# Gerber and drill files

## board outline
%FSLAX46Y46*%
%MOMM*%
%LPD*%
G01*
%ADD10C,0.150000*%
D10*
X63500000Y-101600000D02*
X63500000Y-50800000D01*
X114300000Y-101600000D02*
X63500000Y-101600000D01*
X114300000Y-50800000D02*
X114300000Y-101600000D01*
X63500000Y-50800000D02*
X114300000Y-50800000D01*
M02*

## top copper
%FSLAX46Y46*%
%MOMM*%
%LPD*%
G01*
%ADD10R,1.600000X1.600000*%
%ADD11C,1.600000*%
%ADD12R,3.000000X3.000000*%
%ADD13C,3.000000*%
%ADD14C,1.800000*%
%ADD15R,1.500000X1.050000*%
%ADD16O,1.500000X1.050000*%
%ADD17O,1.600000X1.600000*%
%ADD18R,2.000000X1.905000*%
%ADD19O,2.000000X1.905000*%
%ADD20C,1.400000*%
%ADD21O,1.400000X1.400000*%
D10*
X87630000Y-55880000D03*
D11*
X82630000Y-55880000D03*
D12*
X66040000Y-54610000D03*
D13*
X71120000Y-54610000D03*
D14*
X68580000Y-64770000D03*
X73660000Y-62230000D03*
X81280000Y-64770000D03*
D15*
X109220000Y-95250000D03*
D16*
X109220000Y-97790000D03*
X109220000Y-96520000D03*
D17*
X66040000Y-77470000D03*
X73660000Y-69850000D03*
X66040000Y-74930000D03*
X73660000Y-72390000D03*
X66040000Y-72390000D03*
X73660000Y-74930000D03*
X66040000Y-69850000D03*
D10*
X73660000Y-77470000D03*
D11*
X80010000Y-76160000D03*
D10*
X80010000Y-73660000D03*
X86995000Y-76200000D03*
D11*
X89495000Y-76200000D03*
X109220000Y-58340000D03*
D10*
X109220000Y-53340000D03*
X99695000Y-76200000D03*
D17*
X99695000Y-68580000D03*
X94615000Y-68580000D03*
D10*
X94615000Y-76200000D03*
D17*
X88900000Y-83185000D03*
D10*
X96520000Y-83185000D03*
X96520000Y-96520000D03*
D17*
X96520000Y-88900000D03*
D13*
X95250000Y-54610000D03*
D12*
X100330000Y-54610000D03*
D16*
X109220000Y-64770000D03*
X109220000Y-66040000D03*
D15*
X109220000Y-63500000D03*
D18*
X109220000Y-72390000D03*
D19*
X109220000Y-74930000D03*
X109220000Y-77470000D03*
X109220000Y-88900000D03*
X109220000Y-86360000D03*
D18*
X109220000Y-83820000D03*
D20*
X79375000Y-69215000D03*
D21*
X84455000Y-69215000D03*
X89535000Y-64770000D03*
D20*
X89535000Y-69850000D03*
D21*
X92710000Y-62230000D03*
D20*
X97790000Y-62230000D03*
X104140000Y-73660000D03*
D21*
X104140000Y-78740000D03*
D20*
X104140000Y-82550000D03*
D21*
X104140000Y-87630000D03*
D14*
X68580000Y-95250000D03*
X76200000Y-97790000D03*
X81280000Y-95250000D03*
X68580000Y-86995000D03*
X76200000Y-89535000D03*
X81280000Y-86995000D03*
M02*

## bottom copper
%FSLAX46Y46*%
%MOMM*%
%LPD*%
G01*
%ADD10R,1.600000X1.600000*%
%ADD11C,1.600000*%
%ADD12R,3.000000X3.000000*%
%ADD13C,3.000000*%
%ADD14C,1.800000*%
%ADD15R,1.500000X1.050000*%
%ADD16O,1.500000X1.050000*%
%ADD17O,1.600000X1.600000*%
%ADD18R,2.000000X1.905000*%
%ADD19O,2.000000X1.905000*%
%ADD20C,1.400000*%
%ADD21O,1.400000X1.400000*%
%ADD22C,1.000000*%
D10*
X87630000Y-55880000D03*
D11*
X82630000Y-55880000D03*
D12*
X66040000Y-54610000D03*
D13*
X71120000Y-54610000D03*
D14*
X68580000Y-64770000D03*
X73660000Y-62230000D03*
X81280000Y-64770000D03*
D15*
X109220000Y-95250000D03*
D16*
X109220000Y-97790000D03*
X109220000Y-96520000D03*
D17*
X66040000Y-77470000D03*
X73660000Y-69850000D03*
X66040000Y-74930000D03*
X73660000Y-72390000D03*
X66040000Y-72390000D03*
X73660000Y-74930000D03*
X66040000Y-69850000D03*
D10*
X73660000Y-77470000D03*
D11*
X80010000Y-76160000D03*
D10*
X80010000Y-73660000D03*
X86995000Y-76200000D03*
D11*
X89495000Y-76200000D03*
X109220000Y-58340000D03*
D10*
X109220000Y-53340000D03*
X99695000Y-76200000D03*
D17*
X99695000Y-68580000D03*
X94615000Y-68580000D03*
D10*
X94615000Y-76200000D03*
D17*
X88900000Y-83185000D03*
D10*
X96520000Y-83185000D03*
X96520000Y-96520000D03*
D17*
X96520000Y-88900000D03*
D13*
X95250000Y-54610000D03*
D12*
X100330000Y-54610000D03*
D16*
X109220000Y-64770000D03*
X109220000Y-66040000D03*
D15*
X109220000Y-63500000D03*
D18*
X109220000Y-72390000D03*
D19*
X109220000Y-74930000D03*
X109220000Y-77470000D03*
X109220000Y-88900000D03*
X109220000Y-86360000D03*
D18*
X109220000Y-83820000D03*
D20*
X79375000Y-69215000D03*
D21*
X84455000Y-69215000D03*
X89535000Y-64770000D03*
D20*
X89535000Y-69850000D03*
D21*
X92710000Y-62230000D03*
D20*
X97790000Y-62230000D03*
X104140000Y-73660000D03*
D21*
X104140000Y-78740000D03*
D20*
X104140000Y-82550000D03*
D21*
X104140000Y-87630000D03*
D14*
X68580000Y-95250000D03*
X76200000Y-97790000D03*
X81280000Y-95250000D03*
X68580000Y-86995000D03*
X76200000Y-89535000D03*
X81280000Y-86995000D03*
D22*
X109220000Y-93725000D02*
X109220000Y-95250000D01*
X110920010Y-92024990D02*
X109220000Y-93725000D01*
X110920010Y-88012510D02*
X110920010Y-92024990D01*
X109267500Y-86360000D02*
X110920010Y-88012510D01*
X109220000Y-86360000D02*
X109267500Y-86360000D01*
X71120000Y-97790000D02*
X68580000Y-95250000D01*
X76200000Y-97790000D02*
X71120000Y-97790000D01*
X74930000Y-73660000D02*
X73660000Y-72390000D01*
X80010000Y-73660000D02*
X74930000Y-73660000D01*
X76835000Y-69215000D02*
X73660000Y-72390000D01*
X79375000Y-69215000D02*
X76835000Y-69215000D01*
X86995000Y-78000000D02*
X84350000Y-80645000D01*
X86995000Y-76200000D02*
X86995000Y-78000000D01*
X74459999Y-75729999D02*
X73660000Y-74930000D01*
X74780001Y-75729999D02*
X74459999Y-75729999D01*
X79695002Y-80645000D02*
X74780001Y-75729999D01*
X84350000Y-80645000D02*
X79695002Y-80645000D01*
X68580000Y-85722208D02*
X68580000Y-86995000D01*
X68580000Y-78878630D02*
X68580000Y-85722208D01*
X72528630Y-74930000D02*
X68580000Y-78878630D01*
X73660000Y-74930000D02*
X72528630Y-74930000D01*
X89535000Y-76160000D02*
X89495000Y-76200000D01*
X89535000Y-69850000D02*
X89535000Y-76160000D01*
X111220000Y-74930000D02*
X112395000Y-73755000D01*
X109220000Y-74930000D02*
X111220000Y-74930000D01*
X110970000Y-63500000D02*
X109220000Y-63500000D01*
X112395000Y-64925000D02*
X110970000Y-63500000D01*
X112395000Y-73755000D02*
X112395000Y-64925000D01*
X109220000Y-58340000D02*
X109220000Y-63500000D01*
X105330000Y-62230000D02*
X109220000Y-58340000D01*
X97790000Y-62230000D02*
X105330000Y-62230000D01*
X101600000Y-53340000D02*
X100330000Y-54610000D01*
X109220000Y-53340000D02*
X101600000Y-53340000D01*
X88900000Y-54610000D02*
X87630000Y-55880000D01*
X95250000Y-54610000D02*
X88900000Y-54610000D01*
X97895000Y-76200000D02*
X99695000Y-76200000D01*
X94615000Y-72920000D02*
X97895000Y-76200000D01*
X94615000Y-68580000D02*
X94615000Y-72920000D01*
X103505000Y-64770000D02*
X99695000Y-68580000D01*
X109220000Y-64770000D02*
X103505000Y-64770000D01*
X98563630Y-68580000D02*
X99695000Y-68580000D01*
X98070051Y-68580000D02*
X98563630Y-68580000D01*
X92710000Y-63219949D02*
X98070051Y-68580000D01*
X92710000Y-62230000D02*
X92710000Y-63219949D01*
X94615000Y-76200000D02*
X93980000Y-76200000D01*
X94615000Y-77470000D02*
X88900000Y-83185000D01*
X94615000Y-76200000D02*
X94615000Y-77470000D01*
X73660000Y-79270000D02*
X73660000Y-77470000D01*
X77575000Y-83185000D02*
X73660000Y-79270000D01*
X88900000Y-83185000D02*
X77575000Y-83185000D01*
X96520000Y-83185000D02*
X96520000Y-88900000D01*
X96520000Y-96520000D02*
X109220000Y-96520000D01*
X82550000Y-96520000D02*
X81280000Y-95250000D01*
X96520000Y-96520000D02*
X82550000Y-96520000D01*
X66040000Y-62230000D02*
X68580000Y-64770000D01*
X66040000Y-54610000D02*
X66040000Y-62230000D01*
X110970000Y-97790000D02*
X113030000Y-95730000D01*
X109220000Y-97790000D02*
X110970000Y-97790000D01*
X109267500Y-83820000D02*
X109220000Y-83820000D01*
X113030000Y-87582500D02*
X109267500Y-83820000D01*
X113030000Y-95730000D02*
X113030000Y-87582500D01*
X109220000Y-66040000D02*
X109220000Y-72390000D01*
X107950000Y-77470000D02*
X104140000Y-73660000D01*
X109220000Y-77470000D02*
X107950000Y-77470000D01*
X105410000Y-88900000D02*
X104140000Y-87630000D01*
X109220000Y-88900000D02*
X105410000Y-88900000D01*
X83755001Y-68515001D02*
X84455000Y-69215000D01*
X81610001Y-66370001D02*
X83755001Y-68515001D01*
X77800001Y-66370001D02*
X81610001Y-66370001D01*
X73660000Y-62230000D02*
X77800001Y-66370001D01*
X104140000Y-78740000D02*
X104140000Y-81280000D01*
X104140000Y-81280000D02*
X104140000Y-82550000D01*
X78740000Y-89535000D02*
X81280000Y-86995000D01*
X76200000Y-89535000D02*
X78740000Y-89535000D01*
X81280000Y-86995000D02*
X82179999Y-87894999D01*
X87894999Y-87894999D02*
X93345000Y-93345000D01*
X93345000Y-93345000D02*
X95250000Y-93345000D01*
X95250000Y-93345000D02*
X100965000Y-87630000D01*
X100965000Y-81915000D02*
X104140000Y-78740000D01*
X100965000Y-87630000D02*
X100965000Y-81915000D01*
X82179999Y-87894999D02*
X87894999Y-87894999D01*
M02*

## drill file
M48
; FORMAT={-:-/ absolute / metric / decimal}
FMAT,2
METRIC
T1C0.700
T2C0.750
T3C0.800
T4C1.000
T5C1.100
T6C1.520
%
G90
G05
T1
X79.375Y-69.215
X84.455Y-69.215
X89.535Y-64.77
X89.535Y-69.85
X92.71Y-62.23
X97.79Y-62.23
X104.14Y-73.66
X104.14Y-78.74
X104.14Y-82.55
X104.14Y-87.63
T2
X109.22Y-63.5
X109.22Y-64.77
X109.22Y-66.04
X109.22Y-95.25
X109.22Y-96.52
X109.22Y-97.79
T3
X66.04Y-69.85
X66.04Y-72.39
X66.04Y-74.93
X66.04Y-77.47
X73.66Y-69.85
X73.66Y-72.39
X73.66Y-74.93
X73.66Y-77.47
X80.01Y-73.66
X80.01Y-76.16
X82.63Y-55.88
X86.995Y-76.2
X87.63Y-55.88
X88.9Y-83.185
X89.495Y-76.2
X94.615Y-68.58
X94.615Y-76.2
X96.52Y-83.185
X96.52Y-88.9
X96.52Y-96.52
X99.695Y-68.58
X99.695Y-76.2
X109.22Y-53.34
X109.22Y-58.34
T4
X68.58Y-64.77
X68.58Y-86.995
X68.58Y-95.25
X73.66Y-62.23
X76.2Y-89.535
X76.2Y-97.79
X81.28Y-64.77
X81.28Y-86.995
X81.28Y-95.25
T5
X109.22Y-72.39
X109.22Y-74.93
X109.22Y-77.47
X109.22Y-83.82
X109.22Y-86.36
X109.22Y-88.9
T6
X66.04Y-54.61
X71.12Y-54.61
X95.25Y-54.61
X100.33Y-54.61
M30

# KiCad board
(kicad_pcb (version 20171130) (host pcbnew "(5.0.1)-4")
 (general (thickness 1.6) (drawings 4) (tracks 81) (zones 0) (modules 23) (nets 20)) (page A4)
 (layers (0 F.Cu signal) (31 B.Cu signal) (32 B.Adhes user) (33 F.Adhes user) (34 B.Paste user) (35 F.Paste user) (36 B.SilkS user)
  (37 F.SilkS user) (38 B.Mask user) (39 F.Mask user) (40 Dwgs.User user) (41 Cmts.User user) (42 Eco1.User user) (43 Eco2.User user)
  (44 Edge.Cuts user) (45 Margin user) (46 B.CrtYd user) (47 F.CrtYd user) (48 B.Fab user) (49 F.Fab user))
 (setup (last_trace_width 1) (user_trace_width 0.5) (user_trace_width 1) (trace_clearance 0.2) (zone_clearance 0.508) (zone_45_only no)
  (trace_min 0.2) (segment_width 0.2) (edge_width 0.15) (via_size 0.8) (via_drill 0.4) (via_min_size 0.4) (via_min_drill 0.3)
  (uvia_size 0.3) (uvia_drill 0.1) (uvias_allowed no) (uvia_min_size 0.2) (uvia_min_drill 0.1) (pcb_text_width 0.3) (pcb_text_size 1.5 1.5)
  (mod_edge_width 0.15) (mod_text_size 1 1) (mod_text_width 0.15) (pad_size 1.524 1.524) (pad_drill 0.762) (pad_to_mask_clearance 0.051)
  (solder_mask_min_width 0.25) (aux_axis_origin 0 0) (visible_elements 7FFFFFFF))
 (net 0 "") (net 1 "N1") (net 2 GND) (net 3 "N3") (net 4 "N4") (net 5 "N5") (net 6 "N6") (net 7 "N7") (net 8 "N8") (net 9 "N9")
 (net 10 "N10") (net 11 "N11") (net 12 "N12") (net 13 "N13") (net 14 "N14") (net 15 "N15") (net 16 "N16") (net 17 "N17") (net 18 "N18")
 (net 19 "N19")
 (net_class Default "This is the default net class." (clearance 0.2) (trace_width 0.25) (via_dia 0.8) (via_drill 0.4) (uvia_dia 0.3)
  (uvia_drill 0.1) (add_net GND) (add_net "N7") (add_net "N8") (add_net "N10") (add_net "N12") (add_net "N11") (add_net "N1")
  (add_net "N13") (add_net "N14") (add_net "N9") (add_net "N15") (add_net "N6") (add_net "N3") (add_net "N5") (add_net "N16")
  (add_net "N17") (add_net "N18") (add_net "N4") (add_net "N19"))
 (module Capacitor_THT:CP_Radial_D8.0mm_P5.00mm (layer F.Cu) (at 87.63 55.88 180)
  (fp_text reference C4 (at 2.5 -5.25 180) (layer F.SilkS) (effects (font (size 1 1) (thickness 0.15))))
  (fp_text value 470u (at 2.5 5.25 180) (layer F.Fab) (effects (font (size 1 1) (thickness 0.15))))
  (pad 1 thru_hole rect (at 0 0 180) (size 1.6 1.6) (drill 0.8) (layers *.Cu *.Mask) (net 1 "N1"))
  (pad 2 thru_hole circle (at 5 0 180) (size 1.6 1.6) (drill 0.8) (layers *.Cu *.Mask) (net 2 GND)))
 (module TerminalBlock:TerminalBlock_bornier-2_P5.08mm (layer F.Cu) (at 66.04 54.61)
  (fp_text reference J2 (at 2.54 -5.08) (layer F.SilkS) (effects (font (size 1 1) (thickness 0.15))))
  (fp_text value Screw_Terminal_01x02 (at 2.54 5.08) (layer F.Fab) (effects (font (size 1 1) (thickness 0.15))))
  (pad 1 thru_hole rect (at 0 0) (size 3 3) (drill 1.52) (layers *.Cu *.Mask) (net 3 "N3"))
  (pad 2 thru_hole circle (at 5.08 0) (size 3 3) (drill 1.52) (layers *.Cu *.Mask) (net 2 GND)))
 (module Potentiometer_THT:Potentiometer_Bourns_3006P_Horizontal (layer F.Cu) (at 81.28 64.77)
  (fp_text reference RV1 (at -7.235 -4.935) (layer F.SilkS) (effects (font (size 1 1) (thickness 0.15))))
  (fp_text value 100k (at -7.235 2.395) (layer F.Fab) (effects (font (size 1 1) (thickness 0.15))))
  (pad 3 thru_hole circle (at -12.7 0) (size 1.8 1.8) (drill 1) (layers *.Cu *.Mask) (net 3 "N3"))
  (pad 2 thru_hole circle (at -7.62 -2.54) (size 1.8 1.8) (drill 1) (layers *.Cu *.Mask) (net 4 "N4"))
  (pad 1 thru_hole circle (at 0 0) (size 1.8 1.8) (drill 1) (layers *.Cu *.Mask) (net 2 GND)))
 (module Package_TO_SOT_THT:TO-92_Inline (layer F.Cu) (at 109.22 95.25 270)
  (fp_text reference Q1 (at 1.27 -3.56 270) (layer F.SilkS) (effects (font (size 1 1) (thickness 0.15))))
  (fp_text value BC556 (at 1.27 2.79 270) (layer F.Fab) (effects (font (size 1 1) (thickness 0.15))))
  (pad 1 thru_hole rect (at 0 0 270) (size 1.05 1.5) (drill 0.75) (layers *.Cu *.Mask) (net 2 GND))
  (pad 3 thru_hole oval (at 2.54 0 270) (size 1.05 1.5) (drill 0.75) (layers *.Cu *.Mask) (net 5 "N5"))
  (pad 2 thru_hole oval (at 1.27 0 270) (size 1.05 1.5) (drill 0.75) (layers *.Cu *.Mask) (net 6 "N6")))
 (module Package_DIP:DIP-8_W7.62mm (layer F.Cu) (at 73.66 77.47 180)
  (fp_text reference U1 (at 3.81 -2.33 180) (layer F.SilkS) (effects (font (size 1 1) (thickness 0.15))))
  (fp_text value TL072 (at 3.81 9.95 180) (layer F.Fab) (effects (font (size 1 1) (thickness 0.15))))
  (pad 8 thru_hole oval (at 7.62 0 180) (size 1.6 1.6) (drill 0.8) (layers *.Cu *.Mask))
  (pad 4 thru_hole oval (at 0 7.62 180) (size 1.6 1.6) (drill 0.8) (layers *.Cu *.Mask))
  (pad 7 thru_hole oval (at 7.62 2.54 180) (size 1.6 1.6) (drill 0.8) (layers *.Cu *.Mask))
  (pad 3 thru_hole oval (at 0 5.08 180) (size 1.6 1.6) (drill 0.8) (layers *.Cu *.Mask) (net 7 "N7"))
  (pad 6 thru_hole oval (at 7.62 5.08 180) (size 1.6 1.6) (drill 0.8) (layers *.Cu *.Mask))
  (pad 2 thru_hole oval (at 0 2.54 180) (size 1.6 1.6) (drill 0.8) (layers *.Cu *.Mask) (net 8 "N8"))
  (pad 5 thru_hole oval (at 7.62 7.62 180) (size 1.6 1.6) (drill 0.8) (layers *.Cu *.Mask))
  (pad 1 thru_hole rect (at 0 0 180) (size 1.6 1.6) (drill 0.8) (layers *.Cu *.Mask) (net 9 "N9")))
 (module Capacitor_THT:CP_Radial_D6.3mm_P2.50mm (layer F.Cu) (at 80.01 73.66 270)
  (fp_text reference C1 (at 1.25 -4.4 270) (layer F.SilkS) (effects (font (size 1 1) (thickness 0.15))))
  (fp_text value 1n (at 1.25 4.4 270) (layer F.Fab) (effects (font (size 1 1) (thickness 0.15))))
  (pad 2 thru_hole circle (at 2.5 0 270) (size 1.6 1.6) (drill 0.8) (layers *.Cu *.Mask) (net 2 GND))
  (pad 1 thru_hole rect (at 0 0 270) (size 1.6 1.6) (drill 0.8) (layers *.Cu *.Mask) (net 7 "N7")))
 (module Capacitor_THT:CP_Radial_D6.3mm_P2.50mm (layer F.Cu) (at 86.995 76.2)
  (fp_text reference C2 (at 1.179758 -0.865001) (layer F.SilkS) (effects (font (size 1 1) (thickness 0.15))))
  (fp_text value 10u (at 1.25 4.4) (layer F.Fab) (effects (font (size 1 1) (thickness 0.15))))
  (pad 1 thru_hole rect (at 0 0) (size 1.6 1.6) (drill 0.8) (layers *.Cu *.Mask) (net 8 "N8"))
  (pad 2 thru_hole circle (at 2.5 0) (size 1.6 1.6) (drill 0.8) (layers *.Cu *.Mask) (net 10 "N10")))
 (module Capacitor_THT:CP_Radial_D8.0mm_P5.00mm (layer F.Cu) (at 109.22 53.34 270)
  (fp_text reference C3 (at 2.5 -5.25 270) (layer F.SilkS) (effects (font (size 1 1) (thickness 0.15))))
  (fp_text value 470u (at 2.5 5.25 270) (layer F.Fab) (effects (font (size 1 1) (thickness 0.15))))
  (pad 2 thru_hole circle (at 5 0 270) (size 1.6 1.6) (drill 0.8) (layers *.Cu *.Mask) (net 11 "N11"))
  (pad 1 thru_hole rect (at 0 0 270) (size 1.6 1.6) (drill 0.8) (layers *.Cu *.Mask) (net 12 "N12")))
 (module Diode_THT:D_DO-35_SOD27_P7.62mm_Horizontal (layer F.Cu) (at 99.695 76.2 90)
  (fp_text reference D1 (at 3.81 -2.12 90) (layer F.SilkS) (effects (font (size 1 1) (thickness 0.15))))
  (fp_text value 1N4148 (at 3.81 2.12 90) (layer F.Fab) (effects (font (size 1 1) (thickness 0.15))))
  (pad 1 thru_hole rect (at 0 0 90) (size 1.6 1.6) (drill 0.8) (layers *.Cu *.Mask) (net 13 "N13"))
  (pad 2 thru_hole oval (at 7.62 0 90) (size 1.6 1.6) (drill 0.8) (layers *.Cu *.Mask) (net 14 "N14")))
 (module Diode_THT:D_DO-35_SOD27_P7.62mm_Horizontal (layer F.Cu) (at 94.615 76.2 90)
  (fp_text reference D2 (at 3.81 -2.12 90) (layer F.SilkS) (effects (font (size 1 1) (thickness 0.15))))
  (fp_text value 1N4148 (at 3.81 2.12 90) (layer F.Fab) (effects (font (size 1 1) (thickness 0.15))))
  (pad 2 thru_hole oval (at 7.62 0 90) (size 1.6 1.6) (drill 0.8) (layers *.Cu *.Mask) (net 13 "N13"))
  (pad 1 thru_hole rect (at 0 0 90) (size 1.6 1.6) (drill 0.8) (layers *.Cu *.Mask) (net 9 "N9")))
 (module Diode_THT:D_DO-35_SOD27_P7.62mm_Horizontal (layer F.Cu) (at 96.52 83.185 180)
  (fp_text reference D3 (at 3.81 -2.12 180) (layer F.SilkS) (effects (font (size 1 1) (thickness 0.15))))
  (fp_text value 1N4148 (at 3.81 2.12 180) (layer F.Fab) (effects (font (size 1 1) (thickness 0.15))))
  (pad 2 thru_hole oval (at 7.62 0 180) (size 1.6 1.6) (drill 0.8) (layers *.Cu *.Mask) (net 9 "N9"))
  (pad 1 thru_hole rect (at 0 0 180) (size 1.6 1.6) (drill 0.8) (layers *.Cu *.Mask) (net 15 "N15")))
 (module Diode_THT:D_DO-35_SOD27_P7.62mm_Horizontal (layer F.Cu) (at 96.52 96.52 90)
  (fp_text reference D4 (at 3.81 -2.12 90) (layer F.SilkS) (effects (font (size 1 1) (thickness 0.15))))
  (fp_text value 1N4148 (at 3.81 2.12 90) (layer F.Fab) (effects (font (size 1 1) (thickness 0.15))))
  (pad 1 thru_hole rect (at 0 0 90) (size 1.6 1.6) (drill 0.8) (layers *.Cu *.Mask) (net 6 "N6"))
  (pad 2 thru_hole oval (at 7.62 0 90) (size 1.6 1.6) (drill 0.8) (layers *.Cu *.Mask) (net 15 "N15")))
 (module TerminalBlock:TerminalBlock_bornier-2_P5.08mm (layer F.Cu) (at 100.33 54.61 180)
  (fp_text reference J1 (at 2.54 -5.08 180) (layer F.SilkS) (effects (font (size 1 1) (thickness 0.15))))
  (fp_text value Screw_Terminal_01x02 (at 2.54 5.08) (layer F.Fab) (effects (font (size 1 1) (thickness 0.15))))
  (pad 2 thru_hole circle (at 5.08 0 180) (size 3 3) (drill 1.52) (layers *.Cu *.Mask) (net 1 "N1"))
  (pad 1 thru_hole rect (at 0 0 180) (size 3 3) (drill 1.52) (layers *.Cu *.Mask) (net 12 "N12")))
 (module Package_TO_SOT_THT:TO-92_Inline (layer F.Cu) (at 109.22 63.5 270)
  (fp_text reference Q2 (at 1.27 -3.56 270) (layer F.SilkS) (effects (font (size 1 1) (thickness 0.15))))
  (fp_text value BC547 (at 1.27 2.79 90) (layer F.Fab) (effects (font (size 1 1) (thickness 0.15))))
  (pad 2 thru_hole oval (at 1.27 0 270) (size 1.05 1.5) (drill 0.75) (layers *.Cu *.Mask) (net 14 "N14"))
  (pad 3 thru_hole oval (at 2.54 0 270) (size 1.05 1.5) (drill 0.75) (layers *.Cu *.Mask) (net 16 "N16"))
  (pad 1 thru_hole rect (at 0 0 270) (size 1.05 1.5) (drill 0.75) (layers *.Cu *.Mask) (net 11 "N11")))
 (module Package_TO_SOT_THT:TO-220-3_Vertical (layer F.Cu) (at 109.22 72.39 270)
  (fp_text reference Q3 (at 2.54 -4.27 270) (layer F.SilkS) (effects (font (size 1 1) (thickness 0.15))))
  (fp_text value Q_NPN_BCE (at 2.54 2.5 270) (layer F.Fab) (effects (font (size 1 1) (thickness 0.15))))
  (pad 1 thru_hole rect (at 0 0 270) (size 1.905 2) (drill 1.1) (layers *.Cu *.Mask) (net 16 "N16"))
  (pad 2 thru_hole oval (at 2.54 0 270) (size 1.905 2) (drill 1.1) (layers *.Cu *.Mask) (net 11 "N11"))
  (pad 3 thru_hole oval (at 5.08 0 270) (size 1.905 2) (drill 1.1) (layers *.Cu *.Mask) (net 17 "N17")))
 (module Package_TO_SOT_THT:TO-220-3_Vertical (layer F.Cu) (at 109.22 83.82 270)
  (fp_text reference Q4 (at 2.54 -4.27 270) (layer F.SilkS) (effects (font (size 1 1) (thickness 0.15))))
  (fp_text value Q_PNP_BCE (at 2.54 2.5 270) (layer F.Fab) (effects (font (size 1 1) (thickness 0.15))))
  (pad 3 thru_hole oval (at 5.08 0 270) (size 1.905 2) (drill 1.1) (layers *.Cu *.Mask) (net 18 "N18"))
  (pad 2 thru_hole oval (at 2.54 0 270) (size 1.905 2) (drill 1.1) (layers *.Cu *.Mask) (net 2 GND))
  (pad 1 thru_hole rect (at 0 0 270) (size 1.905 2) (drill 1.1) (layers *.Cu *.Mask) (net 5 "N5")))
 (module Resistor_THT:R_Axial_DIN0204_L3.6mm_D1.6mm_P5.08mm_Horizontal (layer F.Cu) (at 79.375 69.215)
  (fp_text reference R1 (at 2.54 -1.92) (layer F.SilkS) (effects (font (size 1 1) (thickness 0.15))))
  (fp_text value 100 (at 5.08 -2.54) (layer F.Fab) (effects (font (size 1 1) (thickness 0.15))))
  (pad 1 thru_hole circle (at 0 0) (size 1.4 1.4) (drill 0.7) (layers *.Cu *.Mask) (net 7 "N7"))
  (pad 2 thru_hole oval (at 5.08 0) (size 1.4 1.4) (drill 0.7) (layers *.Cu *.Mask) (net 4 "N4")))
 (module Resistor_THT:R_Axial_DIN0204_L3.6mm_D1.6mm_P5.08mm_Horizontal (layer F.Cu) (at 89.535 69.85 90)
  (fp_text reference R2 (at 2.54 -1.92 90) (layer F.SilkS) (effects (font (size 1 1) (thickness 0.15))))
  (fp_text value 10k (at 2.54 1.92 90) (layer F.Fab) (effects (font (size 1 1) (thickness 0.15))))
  (pad 2 thru_hole oval (at 5.08 0 90) (size 1.4 1.4) (drill 0.7) (layers *.Cu *.Mask) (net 2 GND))
  (pad 1 thru_hole circle (at 0 0 90) (size 1.4 1.4) (drill 0.7) (layers *.Cu *.Mask) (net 10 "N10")))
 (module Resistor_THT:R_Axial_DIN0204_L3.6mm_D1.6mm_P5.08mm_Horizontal (layer F.Cu) (at 97.79 62.23 180)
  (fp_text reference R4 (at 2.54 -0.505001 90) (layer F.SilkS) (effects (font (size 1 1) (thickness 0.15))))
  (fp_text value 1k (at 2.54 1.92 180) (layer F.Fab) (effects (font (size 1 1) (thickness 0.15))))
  (pad 2 thru_hole oval (at 5.08 0 180) (size 1.4 1.4) (drill 0.7) (layers *.Cu *.Mask) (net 14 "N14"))
  (pad 1 thru_hole circle (at 0 0 180) (size 1.4 1.4) (drill 0.7) (layers *.Cu *.Mask) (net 11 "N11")))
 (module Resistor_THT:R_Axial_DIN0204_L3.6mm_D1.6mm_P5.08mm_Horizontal (layer F.Cu) (at 104.14 73.66 270)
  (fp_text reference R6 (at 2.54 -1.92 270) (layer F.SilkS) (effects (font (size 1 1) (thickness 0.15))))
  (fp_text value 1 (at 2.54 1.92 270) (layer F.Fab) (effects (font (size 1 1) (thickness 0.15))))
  (pad 1 thru_hole circle (at 0 0 270) (size 1.4 1.4) (drill 0.7) (layers *.Cu *.Mask) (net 17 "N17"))
  (pad 2 thru_hole oval (at 5.08 0 270) (size 1.4 1.4) (drill 0.7) (layers *.Cu *.Mask) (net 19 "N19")))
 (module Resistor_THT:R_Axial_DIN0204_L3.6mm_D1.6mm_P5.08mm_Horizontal (layer F.Cu) (at 104.14 82.55 270)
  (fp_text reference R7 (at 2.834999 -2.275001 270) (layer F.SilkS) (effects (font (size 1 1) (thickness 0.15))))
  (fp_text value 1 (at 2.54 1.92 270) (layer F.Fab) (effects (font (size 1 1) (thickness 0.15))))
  (pad 1 thru_hole circle (at 0 0 270) (size 1.4 1.4) (drill 0.7) (layers *.Cu *.Mask) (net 19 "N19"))
  (pad 2 thru_hole oval (at 5.08 0 270) (size 1.4 1.4) (drill 0.7) (layers *.Cu *.Mask) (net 18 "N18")))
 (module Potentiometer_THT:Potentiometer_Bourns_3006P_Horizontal (layer F.Cu) (at 68.58 95.25 180)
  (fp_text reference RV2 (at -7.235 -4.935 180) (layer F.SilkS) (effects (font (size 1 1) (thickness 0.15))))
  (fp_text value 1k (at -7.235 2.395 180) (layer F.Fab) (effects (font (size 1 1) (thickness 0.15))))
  (pad 1 thru_hole circle (at 0 0 180) (size 1.8 1.8) (drill 1) (layers *.Cu *.Mask) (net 2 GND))
  (pad 2 thru_hole circle (at -7.62 -2.54 180) (size 1.8 1.8) (drill 1) (layers *.Cu *.Mask) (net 2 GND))
  (pad 3 thru_hole circle (at -12.7 0 180) (size 1.8 1.8) (drill 1) (layers *.Cu *.Mask) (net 6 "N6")))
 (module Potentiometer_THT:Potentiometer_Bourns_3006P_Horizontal (layer F.Cu) (at 68.58 86.995 180)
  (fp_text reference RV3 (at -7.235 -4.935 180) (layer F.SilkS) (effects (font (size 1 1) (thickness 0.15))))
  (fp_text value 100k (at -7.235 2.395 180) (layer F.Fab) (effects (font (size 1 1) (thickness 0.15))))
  (pad 1 thru_hole circle (at 0 0 180) (size 1.8 1.8) (drill 1) (layers *.Cu *.Mask) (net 8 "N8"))
  (pad 2 thru_hole circle (at -7.62 -2.54 180) (size 1.8 1.8) (drill 1) (layers *.Cu *.Mask) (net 19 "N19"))
  (pad 3 thru_hole circle (at -12.7 0 180) (size 1.8 1.8) (drill 1) (layers *.Cu *.Mask) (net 19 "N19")))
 (gr_line (start 63.5 101.6) (end 63.5 50.8) (layer Edge.Cuts) (width 0.15))
 (gr_line (start 114.3 101.6) (end 63.5 101.6) (layer Edge.Cuts) (width 0.15))
 (gr_line (start 114.3 50.8) (end 114.3 101.6) (layer Edge.Cuts) (width 0.15))
 (gr_line (start 63.5 50.8) (end 114.3 50.8) (layer Edge.Cuts) (width 0.15))
 (segment (start 109.22 93.725) (end 109.22 95.25) (width 1) (layer B.Cu) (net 2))
 (segment (start 110.92001 92.02499) (end 109.22 93.725) (width 1) (layer B.Cu) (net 2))
 (segment (start 110.92001 88.01251) (end 110.92001 92.02499) (width 1) (layer B.Cu) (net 2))
 (segment (start 109.2675 86.36) (end 110.92001 88.01251) (width 1) (layer B.Cu) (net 2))
 (segment (start 109.22 86.36) (end 109.2675 86.36) (width 1) (layer B.Cu) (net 2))
 (segment (start 71.12 97.79) (end 68.58 95.25) (width 1) (layer B.Cu) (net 2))
 (segment (start 76.2 97.79) (end 71.12 97.79) (width 1) (layer B.Cu) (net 2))
 (segment (start 74.93 73.66) (end 73.66 72.39) (width 1) (layer B.Cu) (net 7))
 (segment (start 80.01 73.66) (end 74.93 73.66) (width 1) (layer B.Cu) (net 7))
 (segment (start 76.835 69.215) (end 73.66 72.39) (width 1) (layer B.Cu) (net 7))
 (segment (start 79.375 69.215) (end 76.835 69.215) (width 1) (layer B.Cu) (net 7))
 (segment (start 86.995 78) (end 84.35 80.645) (width 1) (layer B.Cu) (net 8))
 (segment (start 86.995 76.2) (end 86.995 78) (width 1) (layer B.Cu) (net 8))
 (segment (start 74.459999 75.729999) (end 73.66 74.93) (width 1) (layer B.Cu) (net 8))
 (segment (start 74.780001 75.729999) (end 74.459999 75.729999) (width 1) (layer B.Cu) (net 8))
 (segment (start 79.695002 80.645) (end 74.780001 75.729999) (width 1) (layer B.Cu) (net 8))
 (segment (start 84.35 80.645) (end 79.695002 80.645) (width 1) (layer B.Cu) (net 8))
 (segment (start 68.58 85.722208) (end 68.58 86.995) (width 1) (layer B.Cu) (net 8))
 (segment (start 68.58 78.87863) (end 68.58 85.722208) (width 1) (layer B.Cu) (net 8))
 (segment (start 72.52863 74.93) (end 68.58 78.87863) (width 1) (layer B.Cu) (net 8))
 (segment (start 73.66 74.93) (end 72.52863 74.93) (width 1) (layer B.Cu) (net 8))
 (segment (start 89.535 76.16) (end 89.495 76.2) (width 1) (layer B.Cu) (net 10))
 (segment (start 89.535 69.85) (end 89.535 76.16) (width 1) (layer B.Cu) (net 10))
 (segment (start 111.22 74.93) (end 112.395 73.755) (width 1) (layer B.Cu) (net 11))
 (segment (start 109.22 74.93) (end 111.22 74.93) (width 1) (layer B.Cu) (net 11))
 (segment (start 110.97 63.5) (end 109.22 63.5) (width 1) (layer B.Cu) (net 11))
 (segment (start 112.395 64.925) (end 110.97 63.5) (width 1) (layer B.Cu) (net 11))
 (segment (start 112.395 73.755) (end 112.395 64.925) (width 1) (layer B.Cu) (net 11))
 (segment (start 109.22 58.34) (end 109.22 63.5) (width 1) (layer B.Cu) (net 11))
 (segment (start 105.33 62.23) (end 109.22 58.34) (width 1) (layer B.Cu) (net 11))
 (segment (start 97.79 62.23) (end 105.33 62.23) (width 1) (layer B.Cu) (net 11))
 (segment (start 101.6 53.34) (end 100.33 54.61) (width 1) (layer B.Cu) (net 12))
 (segment (start 109.22 53.34) (end 101.6 53.34) (width 1) (layer B.Cu) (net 12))
 (segment (start 88.9 54.61) (end 87.63 55.88) (width 1) (layer B.Cu) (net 1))
 (segment (start 95.25 54.61) (end 88.9 54.61) (width 1) (layer B.Cu) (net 1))
 (segment (start 97.895 76.2) (end 99.695 76.2) (width 1) (layer B.Cu) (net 13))
 (segment (start 94.615 72.92) (end 97.895 76.2) (width 1) (layer B.Cu) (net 13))
 (segment (start 94.615 68.58) (end 94.615 72.92) (width 1) (layer B.Cu) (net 13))
 (segment (start 103.505 64.77) (end 99.695 68.58) (width 1) (layer B.Cu) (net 14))
 (segment (start 109.22 64.77) (end 103.505 64.77) (width 1) (layer B.Cu) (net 14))
 (segment (start 98.56363 68.58) (end 99.695 68.58) (width 1) (layer B.Cu) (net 14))
 (segment (start 98.070051 68.58) (end 98.56363 68.58) (width 1) (layer B.Cu) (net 14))
 (segment (start 92.71 63.219949) (end 98.070051 68.58) (width 1) (layer B.Cu) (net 14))
 (segment (start 92.71 62.23) (end 92.71 63.219949) (width 1) (layer B.Cu) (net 14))
 (segment (start 94.615 76.2) (end 93.98 76.2) (width 1) (layer B.Cu) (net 9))
 (segment (start 94.615 77.47) (end 88.9 83.185) (width 1) (layer B.Cu) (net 9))
 (segment (start 94.615 76.2) (end 94.615 77.47) (width 1) (layer B.Cu) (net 9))
 (segment (start 73.66 79.27) (end 73.66 77.47) (width 1) (layer B.Cu) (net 9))
 (segment (start 77.575 83.185) (end 73.66 79.27) (width 1) (layer B.Cu) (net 9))
 (segment (start 88.9 83.185) (end 77.575 83.185) (width 1) (layer B.Cu) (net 9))
 (segment (start 96.52 83.185) (end 96.52 88.9) (width 1) (layer B.Cu) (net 15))
 (segment (start 96.52 96.52) (end 109.22 96.52) (width 1) (layer B.Cu) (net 6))
 (segment (start 82.55 96.52) (end 81.28 95.25) (width 1) (layer B.Cu) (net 6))
 (segment (start 96.52 96.52) (end 82.55 96.52) (width 1) (layer B.Cu) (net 6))
 (segment (start 66.04 62.23) (end 68.58 64.77) (width 1) (layer B.Cu) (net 3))
 (segment (start 66.04 54.61) (end 66.04 62.23) (width 1) (layer B.Cu) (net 3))
 (segment (start 110.97 97.79) (end 113.03 95.73) (width 1) (layer B.Cu) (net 5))
 (segment (start 109.22 97.79) (end 110.97 97.79) (width 1) (layer B.Cu) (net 5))
 (segment (start 109.2675 83.82) (end 109.22 83.82) (width 1) (layer B.Cu) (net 5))
 (segment (start 113.03 87.5825) (end 109.2675 83.82) (width 1) (layer B.Cu) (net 5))
 (segment (start 113.03 95.73) (end 113.03 87.5825) (width 1) (layer B.Cu) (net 5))
 (segment (start 109.22 66.04) (end 109.22 72.39) (width 1) (layer B.Cu) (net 16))
 (segment (start 107.95 77.47) (end 104.14 73.66) (width 1) (layer B.Cu) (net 17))
 (segment (start 109.22 77.47) (end 107.95 77.47) (width 1) (layer B.Cu) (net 17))
 (segment (start 105.41 88.9) (end 104.14 87.63) (width 1) (layer B.Cu) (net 18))
 (segment (start 109.22 88.9) (end 105.41 88.9) (width 1) (layer B.Cu) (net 18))
 (segment (start 83.755001 68.515001) (end 84.455 69.215) (width 1) (layer B.Cu) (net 4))
 (segment (start 81.610001 66.370001) (end 83.755001 68.515001) (width 1) (layer B.Cu) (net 4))
 (segment (start 77.800001 66.370001) (end 81.610001 66.370001) (width 1) (layer B.Cu) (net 4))
 (segment (start 73.66 62.23) (end 77.800001 66.370001) (width 1) (layer B.Cu) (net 4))
 (segment (start 104.14 78.74) (end 104.14 81.28) (width 1) (layer B.Cu) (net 19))
 (segment (start 104.14 81.28) (end 104.14 82.55) (width 1) (layer B.Cu) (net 19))
 (segment (start 78.74 89.535) (end 81.28 86.995) (width 1) (layer B.Cu) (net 19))
 (segment (start 76.2 89.535) (end 78.74 89.535) (width 1) (layer B.Cu) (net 19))
 (segment (start 81.28 86.995) (end 82.179999 87.894999) (width 1) (layer B.Cu) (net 19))
 (segment (start 87.894999 87.894999) (end 93.345 93.345) (width 1) (layer B.Cu) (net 19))
 (segment (start 93.345 93.345) (end 95.25 93.345) (width 1) (layer B.Cu) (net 19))
 (segment (start 95.25 93.345) (end 100.965 87.63) (width 1) (layer B.Cu) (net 19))
 (segment (start 100.965 81.915) (end 104.14 78.74) (width 1) (layer B.Cu) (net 19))
 (segment (start 100.965 87.63) (end 100.965 81.915) (width 1) (layer B.Cu) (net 19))
 (segment (start 82.179999 87.894999) (end 87.894999 87.894999) (width 1) (layer B.Cu) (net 19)))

